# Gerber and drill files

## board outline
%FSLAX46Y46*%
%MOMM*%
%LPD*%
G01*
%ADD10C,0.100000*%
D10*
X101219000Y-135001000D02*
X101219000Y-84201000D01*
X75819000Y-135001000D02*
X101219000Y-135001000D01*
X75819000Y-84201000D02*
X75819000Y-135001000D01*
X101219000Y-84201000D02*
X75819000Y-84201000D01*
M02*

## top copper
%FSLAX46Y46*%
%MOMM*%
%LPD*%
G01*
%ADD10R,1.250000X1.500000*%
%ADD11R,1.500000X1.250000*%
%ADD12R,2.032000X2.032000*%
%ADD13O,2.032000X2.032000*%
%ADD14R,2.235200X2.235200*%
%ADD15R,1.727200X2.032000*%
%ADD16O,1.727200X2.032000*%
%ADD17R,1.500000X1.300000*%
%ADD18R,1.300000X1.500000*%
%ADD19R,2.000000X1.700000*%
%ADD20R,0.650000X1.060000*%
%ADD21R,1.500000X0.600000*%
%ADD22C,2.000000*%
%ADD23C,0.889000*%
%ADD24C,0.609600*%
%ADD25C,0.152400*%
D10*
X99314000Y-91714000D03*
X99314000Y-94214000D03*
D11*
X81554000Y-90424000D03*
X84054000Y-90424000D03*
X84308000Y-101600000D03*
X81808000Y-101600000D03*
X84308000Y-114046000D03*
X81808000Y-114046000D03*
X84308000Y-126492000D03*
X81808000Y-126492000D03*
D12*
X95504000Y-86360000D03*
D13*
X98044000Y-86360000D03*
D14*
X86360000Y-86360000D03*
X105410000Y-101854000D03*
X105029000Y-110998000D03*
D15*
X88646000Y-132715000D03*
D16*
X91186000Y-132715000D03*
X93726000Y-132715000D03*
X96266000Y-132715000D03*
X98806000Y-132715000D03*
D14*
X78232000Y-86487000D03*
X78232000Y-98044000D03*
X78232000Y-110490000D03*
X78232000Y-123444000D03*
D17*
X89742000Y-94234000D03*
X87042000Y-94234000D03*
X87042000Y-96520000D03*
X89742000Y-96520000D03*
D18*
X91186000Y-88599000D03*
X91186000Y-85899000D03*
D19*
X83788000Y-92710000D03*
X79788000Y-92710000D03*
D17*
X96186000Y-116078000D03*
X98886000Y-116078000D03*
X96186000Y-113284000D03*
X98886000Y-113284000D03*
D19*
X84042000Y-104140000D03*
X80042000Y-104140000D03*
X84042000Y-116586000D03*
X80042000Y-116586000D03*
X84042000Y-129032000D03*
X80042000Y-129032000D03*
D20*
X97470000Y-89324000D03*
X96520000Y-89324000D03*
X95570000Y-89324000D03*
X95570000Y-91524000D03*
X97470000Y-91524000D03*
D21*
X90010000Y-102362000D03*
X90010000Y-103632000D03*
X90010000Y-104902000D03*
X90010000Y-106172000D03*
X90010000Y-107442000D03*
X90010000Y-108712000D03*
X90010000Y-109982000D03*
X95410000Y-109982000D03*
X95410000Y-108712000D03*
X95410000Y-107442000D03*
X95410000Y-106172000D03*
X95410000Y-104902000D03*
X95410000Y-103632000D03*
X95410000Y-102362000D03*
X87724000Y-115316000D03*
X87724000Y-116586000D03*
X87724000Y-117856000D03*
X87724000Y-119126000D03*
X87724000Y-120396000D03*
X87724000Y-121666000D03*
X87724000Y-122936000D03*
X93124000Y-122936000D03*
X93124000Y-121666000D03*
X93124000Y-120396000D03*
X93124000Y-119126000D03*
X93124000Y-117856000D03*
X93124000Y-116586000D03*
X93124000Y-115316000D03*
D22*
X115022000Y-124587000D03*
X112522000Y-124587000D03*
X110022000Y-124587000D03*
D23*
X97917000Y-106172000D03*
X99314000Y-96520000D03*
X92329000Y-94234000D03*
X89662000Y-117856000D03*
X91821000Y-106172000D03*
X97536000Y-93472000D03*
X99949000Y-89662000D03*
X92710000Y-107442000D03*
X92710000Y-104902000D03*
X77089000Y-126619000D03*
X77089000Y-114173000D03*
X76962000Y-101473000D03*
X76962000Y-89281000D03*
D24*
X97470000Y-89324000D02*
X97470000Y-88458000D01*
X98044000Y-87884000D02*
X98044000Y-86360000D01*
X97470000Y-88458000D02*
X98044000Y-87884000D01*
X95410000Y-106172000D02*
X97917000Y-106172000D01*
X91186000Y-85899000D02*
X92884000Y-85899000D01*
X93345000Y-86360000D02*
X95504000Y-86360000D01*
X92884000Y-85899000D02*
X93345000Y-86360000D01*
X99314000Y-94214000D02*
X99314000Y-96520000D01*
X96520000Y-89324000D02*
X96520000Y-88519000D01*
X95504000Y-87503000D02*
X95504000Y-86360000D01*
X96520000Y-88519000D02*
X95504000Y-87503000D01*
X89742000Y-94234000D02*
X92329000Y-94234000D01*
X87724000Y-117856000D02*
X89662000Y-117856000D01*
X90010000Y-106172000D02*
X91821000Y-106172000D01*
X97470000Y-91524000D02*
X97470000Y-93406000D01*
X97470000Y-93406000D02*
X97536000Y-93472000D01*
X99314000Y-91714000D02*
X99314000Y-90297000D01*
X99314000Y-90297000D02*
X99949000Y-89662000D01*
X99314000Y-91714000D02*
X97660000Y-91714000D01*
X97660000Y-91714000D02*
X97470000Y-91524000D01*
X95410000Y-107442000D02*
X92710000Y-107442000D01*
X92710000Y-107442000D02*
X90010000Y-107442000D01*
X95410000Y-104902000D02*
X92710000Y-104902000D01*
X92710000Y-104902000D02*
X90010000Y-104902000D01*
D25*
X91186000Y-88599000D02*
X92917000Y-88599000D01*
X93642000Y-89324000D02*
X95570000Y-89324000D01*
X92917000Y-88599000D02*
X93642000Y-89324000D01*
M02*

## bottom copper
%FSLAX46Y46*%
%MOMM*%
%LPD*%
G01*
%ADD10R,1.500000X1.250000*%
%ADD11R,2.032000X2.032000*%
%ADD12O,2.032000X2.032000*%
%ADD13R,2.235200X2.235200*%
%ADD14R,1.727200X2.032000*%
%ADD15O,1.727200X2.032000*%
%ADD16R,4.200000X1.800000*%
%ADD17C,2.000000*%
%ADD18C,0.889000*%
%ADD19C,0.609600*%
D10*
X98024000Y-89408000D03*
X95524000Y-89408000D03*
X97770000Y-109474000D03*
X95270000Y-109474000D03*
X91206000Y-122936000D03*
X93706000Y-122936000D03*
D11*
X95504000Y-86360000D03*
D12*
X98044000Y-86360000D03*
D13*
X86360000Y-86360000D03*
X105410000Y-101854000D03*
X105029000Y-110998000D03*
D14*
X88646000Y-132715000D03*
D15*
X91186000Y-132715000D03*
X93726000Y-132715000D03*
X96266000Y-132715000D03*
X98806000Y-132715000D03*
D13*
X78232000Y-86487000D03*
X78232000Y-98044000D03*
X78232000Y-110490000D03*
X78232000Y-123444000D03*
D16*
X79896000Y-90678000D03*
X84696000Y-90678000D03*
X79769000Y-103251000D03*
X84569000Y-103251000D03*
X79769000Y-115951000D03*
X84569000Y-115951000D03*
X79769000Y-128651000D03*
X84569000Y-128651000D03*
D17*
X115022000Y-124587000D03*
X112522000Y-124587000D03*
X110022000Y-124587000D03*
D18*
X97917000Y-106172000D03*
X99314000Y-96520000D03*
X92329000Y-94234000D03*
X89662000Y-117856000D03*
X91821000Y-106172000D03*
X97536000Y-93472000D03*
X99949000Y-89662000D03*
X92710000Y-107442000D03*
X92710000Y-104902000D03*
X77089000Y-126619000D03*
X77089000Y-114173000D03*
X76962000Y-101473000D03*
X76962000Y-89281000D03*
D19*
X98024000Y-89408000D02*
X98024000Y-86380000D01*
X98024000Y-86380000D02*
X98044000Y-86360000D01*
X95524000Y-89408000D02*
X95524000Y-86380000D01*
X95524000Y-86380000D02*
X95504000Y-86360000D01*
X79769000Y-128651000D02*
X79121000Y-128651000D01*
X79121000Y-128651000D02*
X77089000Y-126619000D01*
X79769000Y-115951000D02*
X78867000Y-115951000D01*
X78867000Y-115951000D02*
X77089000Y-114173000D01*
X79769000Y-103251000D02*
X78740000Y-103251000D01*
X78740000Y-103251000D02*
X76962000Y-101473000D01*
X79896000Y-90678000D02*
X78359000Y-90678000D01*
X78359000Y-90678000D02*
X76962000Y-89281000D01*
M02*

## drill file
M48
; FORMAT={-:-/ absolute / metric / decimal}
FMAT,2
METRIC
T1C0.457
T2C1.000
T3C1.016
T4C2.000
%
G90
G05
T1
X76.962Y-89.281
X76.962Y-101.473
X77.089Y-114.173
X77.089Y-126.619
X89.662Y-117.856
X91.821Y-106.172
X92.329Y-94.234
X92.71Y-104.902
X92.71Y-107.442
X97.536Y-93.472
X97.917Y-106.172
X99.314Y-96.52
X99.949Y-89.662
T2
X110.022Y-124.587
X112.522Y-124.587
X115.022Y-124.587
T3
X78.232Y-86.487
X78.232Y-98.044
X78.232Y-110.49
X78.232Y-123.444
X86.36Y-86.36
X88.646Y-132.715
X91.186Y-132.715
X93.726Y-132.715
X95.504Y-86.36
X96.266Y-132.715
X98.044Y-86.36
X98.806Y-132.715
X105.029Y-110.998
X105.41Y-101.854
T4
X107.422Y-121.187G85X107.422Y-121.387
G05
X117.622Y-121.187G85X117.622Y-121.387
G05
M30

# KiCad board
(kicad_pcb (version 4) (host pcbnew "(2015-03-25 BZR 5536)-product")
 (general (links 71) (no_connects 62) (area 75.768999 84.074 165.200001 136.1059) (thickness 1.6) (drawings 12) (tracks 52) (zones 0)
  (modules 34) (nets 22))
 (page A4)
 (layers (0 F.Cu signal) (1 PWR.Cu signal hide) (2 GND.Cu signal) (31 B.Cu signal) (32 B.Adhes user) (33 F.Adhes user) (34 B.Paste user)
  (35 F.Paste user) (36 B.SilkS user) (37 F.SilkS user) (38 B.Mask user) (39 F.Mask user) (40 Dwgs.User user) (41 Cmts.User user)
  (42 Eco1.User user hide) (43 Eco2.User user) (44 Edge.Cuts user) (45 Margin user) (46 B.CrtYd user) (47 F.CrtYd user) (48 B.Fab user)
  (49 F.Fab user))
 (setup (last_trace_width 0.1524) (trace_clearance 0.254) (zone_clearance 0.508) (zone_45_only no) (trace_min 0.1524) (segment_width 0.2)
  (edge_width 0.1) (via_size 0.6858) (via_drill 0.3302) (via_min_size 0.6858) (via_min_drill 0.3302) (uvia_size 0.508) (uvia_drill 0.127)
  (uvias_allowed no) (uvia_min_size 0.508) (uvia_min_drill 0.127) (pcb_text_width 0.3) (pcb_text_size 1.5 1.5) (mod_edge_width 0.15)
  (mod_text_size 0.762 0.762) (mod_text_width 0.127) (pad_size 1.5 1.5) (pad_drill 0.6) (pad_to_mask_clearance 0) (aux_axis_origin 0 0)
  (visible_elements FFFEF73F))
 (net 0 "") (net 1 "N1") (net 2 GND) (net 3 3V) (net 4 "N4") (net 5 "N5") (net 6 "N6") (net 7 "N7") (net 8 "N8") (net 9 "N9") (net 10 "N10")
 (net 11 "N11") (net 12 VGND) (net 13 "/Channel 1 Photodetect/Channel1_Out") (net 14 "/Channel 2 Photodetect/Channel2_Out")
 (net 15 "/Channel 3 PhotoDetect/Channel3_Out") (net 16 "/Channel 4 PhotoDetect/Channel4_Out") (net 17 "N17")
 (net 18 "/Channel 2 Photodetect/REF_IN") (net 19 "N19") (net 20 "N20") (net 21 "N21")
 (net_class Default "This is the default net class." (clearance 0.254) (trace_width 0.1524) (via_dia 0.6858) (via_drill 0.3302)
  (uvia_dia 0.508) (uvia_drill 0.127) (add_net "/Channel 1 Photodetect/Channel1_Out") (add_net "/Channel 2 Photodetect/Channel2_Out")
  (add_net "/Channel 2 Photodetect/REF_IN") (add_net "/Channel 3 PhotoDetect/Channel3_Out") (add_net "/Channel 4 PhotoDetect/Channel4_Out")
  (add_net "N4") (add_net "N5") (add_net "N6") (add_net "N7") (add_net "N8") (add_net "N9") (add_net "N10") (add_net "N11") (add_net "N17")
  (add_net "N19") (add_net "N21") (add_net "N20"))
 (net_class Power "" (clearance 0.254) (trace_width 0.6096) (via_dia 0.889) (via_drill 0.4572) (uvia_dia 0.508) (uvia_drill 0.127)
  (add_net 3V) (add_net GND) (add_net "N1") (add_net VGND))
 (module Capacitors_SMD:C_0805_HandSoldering (layer B.Cu) (at 96.774 89.408 180)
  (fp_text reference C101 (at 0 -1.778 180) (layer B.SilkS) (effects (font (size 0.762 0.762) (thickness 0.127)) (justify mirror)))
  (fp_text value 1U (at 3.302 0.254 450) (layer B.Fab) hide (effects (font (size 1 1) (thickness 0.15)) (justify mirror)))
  (pad 1 smd rect (at -1.25 0 180) (size 1.5 1.25) (layers B.Cu B.Paste B.Mask) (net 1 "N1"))
  (pad 2 smd rect (at 1.25 0 180) (size 1.5 1.25) (layers B.Cu B.Paste B.Mask) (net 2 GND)))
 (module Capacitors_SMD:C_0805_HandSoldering (layer F.Cu) (at 99.314 92.964 270)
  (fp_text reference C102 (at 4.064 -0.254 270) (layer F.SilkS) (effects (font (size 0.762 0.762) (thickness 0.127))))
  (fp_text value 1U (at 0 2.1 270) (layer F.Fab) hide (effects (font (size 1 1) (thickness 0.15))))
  (pad 1 smd rect (at -1.25 0 270) (size 1.5 1.25) (layers F.Cu F.Paste F.Mask) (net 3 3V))
  (pad 2 smd rect (at 1.25 0 270) (size 1.5 1.25) (layers F.Cu F.Paste F.Mask) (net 2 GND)))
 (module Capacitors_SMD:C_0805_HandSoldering (layer F.Cu) (at 82.804 90.424)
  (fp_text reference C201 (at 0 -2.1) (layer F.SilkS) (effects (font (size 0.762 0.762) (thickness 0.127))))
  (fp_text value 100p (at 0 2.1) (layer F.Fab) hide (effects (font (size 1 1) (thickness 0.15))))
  (pad 1 smd rect (at -1.25 0) (size 1.5 1.25) (layers F.Cu F.Paste F.Mask) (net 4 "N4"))
  (pad 2 smd rect (at 1.25 0) (size 1.5 1.25) (layers F.Cu F.Paste F.Mask) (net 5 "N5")))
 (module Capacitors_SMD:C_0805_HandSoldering (layer B.Cu) (at 96.52 109.474 180)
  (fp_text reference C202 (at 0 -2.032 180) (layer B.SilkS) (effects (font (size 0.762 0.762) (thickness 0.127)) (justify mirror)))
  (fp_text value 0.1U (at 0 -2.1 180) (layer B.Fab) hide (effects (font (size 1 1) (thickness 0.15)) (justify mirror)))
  (pad 1 smd rect (at -1.25 0 180) (size 1.5 1.25) (layers B.Cu B.Paste B.Mask) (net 2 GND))
  (pad 2 smd rect (at 1.25 0 180) (size 1.5 1.25) (layers B.Cu B.Paste B.Mask) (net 3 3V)))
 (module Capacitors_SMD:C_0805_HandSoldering (layer B.Cu) (at 92.456 122.936)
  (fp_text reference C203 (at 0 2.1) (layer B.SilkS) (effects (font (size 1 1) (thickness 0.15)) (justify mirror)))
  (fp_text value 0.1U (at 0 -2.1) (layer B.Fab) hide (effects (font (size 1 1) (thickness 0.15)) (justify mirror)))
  (pad 1 smd rect (at -1.25 0) (size 1.5 1.25) (layers B.Cu B.Paste B.Mask) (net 2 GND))
  (pad 2 smd rect (at 1.25 0) (size 1.5 1.25) (layers B.Cu B.Paste B.Mask) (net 3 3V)))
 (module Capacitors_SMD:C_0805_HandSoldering (layer F.Cu) (at 83.058 101.6 180)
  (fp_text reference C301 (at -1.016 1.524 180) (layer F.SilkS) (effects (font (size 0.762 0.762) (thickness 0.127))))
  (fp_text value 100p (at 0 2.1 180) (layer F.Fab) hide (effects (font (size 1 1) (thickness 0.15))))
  (pad 1 smd rect (at -1.25 0 180) (size 1.5 1.25) (layers F.Cu F.Paste F.Mask) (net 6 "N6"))
  (pad 2 smd rect (at 1.25 0 180) (size 1.5 1.25) (layers F.Cu F.Paste F.Mask) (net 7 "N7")))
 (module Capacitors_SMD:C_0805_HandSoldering (layer F.Cu) (at 83.058 114.046 180)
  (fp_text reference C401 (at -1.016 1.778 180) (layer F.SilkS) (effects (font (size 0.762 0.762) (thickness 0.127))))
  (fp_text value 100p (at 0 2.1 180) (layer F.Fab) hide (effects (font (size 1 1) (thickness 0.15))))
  (pad 1 smd rect (at -1.25 0 180) (size 1.5 1.25) (layers F.Cu F.Paste F.Mask) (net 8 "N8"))
  (pad 2 smd rect (at 1.25 0 180) (size 1.5 1.25) (layers F.Cu F.Paste F.Mask) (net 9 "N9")))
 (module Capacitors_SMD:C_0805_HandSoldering (layer F.Cu) (at 83.058 126.492 180)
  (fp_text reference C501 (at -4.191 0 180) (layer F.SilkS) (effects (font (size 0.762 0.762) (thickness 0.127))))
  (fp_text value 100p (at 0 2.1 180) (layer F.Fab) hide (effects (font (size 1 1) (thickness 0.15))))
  (pad 1 smd rect (at -1.25 0 180) (size 1.5 1.25) (layers F.Cu F.Paste F.Mask) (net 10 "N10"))
  (pad 2 smd rect (at 1.25 0 180) (size 1.5 1.25) (layers F.Cu F.Paste F.Mask) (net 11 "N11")))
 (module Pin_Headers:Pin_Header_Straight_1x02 (layer F.Cu) (at 95.504 86.36 90)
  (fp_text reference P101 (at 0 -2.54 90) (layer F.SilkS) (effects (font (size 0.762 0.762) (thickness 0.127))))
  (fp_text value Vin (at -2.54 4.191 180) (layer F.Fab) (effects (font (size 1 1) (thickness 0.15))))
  (pad 1 thru_hole rect (at 0 0 90) (size 2.032 2.032) (drill 1.016) (layers *.Cu *.Mask F.SilkS) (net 2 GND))
  (pad 2 thru_hole oval (at 0 2.54 90) (size 2.032 2.032) (drill 1.016) (layers *.Cu *.Mask F.SilkS) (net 1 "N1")))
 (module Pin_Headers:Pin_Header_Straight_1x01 (layer F.Cu) (at 86.36 86.36)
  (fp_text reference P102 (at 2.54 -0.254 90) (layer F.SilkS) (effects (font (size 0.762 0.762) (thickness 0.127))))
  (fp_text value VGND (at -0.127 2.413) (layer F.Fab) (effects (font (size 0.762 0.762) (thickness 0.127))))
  (pad 1 thru_hole rect (at 0 0) (size 2.2352 2.2352) (drill 1.016) (layers *.Cu *.Mask F.SilkS) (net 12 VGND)))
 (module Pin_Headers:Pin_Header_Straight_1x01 (layer F.Cu) (at 105.41 101.854)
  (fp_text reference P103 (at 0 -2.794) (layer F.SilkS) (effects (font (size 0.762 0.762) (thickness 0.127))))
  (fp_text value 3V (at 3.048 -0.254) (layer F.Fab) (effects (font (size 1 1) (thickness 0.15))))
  (pad 1 thru_hole rect (at 0 0) (size 2.2352 2.2352) (drill 1.016) (layers *.Cu *.Mask F.SilkS) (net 3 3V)))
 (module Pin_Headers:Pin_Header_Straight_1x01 (layer F.Cu) (at 105.029 110.998)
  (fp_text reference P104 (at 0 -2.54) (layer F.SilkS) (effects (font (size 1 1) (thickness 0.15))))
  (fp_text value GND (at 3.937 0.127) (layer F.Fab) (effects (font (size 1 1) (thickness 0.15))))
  (pad 1 thru_hole rect (at 0 0) (size 2.2352 2.2352) (drill 1.016) (layers *.Cu *.Mask F.SilkS) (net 2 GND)))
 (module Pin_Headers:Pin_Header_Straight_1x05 (layer F.Cu) (at 88.646 132.715 90)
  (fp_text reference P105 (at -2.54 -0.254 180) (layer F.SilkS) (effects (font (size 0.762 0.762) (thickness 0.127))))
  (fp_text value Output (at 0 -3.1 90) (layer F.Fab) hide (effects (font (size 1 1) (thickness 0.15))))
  (pad 1 thru_hole rect (at 0 0 90) (size 2.032 1.7272) (drill 1.016) (layers *.Cu *.Mask F.SilkS)
   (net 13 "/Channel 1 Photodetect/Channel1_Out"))
  (pad 2 thru_hole oval (at 0 2.54 90) (size 2.032 1.7272) (drill 1.016) (layers *.Cu *.Mask F.SilkS)
   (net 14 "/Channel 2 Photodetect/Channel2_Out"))
  (pad 3 thru_hole oval (at 0 5.08 90) (size 2.032 1.7272) (drill 1.016) (layers *.Cu *.Mask F.SilkS)
   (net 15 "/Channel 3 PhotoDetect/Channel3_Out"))
  (pad 4 thru_hole oval (at 0 7.62 90) (size 2.032 1.7272) (drill 1.016) (layers *.Cu *.Mask F.SilkS)
   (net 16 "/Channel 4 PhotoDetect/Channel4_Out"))
  (pad 5 thru_hole oval (at 0 10.16 90) (size 2.032 1.7272) (drill 1.016) (layers *.Cu *.Mask F.SilkS) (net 2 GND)))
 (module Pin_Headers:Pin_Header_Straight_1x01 (layer F.Cu) (at 78.232 86.487)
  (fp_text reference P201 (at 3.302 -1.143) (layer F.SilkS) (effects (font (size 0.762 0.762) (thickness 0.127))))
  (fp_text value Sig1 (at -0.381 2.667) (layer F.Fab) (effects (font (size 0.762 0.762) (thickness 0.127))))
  (pad 1 thru_hole rect (at 0 0) (size 2.2352 2.2352) (drill 1.016) (layers *.Cu *.Mask F.SilkS) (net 4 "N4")))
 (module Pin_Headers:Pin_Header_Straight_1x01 (layer F.Cu) (at 78.232 98.044)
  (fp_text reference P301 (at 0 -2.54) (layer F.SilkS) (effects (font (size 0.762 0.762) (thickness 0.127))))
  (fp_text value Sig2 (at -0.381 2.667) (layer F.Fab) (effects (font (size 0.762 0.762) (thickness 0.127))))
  (pad 1 thru_hole rect (at 0 0) (size 2.2352 2.2352) (drill 1.016) (layers *.Cu *.Mask F.SilkS) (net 6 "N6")))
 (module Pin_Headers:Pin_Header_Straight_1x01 (layer F.Cu) (at 78.232 110.49)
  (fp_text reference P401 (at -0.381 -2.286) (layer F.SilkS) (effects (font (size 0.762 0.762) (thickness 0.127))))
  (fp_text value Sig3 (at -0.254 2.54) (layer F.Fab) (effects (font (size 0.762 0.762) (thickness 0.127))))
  (pad 1 thru_hole rect (at 0 0) (size 2.2352 2.2352) (drill 1.016) (layers *.Cu *.Mask F.SilkS) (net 8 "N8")))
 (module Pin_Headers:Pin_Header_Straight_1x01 (layer F.Cu) (at 78.232 123.444)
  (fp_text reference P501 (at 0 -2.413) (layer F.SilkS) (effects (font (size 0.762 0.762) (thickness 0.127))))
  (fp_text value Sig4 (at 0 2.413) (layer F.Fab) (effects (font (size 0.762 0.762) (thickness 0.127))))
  (pad 1 thru_hole rect (at 0 0) (size 2.2352 2.2352) (drill 1.016) (layers *.Cu *.Mask F.SilkS) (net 10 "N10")))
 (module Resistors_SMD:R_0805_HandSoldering (layer F.Cu) (at 88.392 94.234 180)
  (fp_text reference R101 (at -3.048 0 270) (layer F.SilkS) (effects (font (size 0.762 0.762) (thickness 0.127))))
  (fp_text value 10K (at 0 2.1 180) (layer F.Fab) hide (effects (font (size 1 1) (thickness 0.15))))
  (pad 1 smd rect (at -1.35 0 180) (size 1.5 1.3) (layers F.Cu F.Paste F.Mask) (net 3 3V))
  (pad 2 smd rect (at 1.35 0 180) (size 1.5 1.3) (layers F.Cu F.Paste F.Mask) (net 12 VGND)))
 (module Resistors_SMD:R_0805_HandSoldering (layer F.Cu) (at 88.392 96.52)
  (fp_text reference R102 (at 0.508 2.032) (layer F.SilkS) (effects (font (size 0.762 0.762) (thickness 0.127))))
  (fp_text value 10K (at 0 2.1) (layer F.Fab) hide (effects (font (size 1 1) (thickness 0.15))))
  (pad 1 smd rect (at -1.35 0) (size 1.5 1.3) (layers F.Cu F.Paste F.Mask) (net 12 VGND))
  (pad 2 smd rect (at 1.35 0) (size 1.5 1.3) (layers F.Cu F.Paste F.Mask) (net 2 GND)))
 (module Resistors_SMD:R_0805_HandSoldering (layer F.Cu) (at 91.186 87.249 90)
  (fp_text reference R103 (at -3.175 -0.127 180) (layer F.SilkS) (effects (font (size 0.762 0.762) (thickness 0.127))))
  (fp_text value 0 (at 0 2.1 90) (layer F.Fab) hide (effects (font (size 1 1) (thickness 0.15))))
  (pad 1 smd rect (at -1.35 0 90) (size 1.5 1.3) (layers F.Cu F.Paste F.Mask) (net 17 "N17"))
  (pad 2 smd rect (at 1.35 0 90) (size 1.5 1.3) (layers F.Cu F.Paste F.Mask) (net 2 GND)))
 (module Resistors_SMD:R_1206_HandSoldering (layer F.Cu) (at 81.788 92.71 180)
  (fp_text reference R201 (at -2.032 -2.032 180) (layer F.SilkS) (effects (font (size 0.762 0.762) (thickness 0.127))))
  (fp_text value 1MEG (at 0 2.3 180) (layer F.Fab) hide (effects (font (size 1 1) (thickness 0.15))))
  (pad 1 smd rect (at -2 0 180) (size 2 1.7) (layers F.Cu F.Paste F.Mask) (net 4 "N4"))
  (pad 2 smd rect (at 2 0 180) (size 2 1.7) (layers F.Cu F.Paste F.Mask) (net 5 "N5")))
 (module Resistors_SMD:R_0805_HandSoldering (layer F.Cu) (at 97.536 116.078)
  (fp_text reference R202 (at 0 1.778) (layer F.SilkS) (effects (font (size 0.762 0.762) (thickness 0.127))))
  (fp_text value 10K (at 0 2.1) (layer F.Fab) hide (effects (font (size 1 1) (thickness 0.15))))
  (pad 1 smd rect (at -1.35 0) (size 1.5 1.3) (layers F.Cu F.Paste F.Mask) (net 2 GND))
  (pad 2 smd rect (at 1.35 0) (size 1.5 1.3) (layers F.Cu F.Paste F.Mask) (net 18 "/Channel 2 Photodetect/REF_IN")))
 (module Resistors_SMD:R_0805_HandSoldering (layer F.Cu) (at 97.536 113.284)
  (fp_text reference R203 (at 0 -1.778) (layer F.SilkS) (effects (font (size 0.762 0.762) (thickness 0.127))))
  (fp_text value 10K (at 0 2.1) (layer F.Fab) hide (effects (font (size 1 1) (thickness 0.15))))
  (pad 1 smd rect (at -1.35 0) (size 1.5 1.3) (layers F.Cu F.Paste F.Mask) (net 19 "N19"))
  (pad 2 smd rect (at 1.35 0) (size 1.5 1.3) (layers F.Cu F.Paste F.Mask) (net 3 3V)))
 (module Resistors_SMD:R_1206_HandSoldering (layer F.Cu) (at 82.042 104.14 180)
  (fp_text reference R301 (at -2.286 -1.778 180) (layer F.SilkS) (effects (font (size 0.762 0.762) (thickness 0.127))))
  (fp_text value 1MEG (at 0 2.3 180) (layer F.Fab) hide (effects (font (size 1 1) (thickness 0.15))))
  (pad 1 smd rect (at -2 0 180) (size 2 1.7) (layers F.Cu F.Paste F.Mask) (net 6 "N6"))
  (pad 2 smd rect (at 2 0 180) (size 2 1.7) (layers F.Cu F.Paste F.Mask) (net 7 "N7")))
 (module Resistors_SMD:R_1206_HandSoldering (layer F.Cu) (at 82.042 116.586 180)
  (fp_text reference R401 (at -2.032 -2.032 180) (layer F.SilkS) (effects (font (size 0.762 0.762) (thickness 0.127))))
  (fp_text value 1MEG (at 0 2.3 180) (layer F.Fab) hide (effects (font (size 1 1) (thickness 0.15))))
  (pad 1 smd rect (at -2 0 180) (size 2 1.7) (layers F.Cu F.Paste F.Mask) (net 8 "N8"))
  (pad 2 smd rect (at 2 0 180) (size 2 1.7) (layers F.Cu F.Paste F.Mask) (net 9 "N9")))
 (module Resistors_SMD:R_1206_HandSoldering (layer F.Cu) (at 82.042 129.032 180)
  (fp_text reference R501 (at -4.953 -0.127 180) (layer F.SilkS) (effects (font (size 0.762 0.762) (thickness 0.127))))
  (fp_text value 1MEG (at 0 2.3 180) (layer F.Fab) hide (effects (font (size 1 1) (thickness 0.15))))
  (pad 1 smd rect (at -2 0 180) (size 2 1.7) (layers F.Cu F.Paste F.Mask) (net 10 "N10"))
  (pad 2 smd rect (at 2 0 180) (size 2 1.7) (layers F.Cu F.Paste F.Mask) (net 11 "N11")))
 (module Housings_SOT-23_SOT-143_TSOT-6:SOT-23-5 (layer F.Cu) (at 96.52 90.424 270)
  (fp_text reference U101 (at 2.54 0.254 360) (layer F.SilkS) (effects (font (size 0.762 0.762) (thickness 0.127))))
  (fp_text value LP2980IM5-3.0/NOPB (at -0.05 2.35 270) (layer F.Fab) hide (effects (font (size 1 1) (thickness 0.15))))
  (pad 1 smd rect (at -1.1 -0.95 270) (size 1.06 0.65) (layers F.Cu F.Paste F.Mask) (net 1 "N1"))
  (pad 2 smd rect (at -1.1 0 270) (size 1.06 0.65) (layers F.Cu F.Paste F.Mask) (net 2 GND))
  (pad 3 smd rect (at -1.1 0.95 270) (size 1.06 0.65) (layers F.Cu F.Paste F.Mask) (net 17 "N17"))
  (pad 4 smd rect (at 1.1 0.95 270) (size 1.06 0.65) (layers F.Cu F.Paste F.Mask) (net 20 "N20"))
  (pad 5 smd rect (at 1.1 -0.95 270) (size 1.06 0.65) (layers F.Cu F.Paste F.Mask) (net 3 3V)))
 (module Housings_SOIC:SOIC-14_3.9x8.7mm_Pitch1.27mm (layer F.Cu) (at 92.71 106.172)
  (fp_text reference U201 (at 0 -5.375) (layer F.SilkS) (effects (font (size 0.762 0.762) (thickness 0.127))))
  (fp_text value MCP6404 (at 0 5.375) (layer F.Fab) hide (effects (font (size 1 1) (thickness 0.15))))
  (pad 1 smd rect (at -2.7 -3.81) (size 1.5 0.6) (layers F.Cu F.Paste F.Mask) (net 4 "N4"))
  (pad 2 smd rect (at -2.7 -2.54) (size 1.5 0.6) (layers F.Cu F.Paste F.Mask) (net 5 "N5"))
  (pad 3 smd rect (at -2.7 -1.27) (size 1.5 0.6) (layers F.Cu F.Paste F.Mask) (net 12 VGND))
  (pad 4 smd rect (at -2.7 0) (size 1.5 0.6) (layers F.Cu F.Paste F.Mask) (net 3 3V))
  (pad 5 smd rect (at -2.7 1.27) (size 1.5 0.6) (layers F.Cu F.Paste F.Mask) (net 12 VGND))
  (pad 6 smd rect (at -2.7 2.54) (size 1.5 0.6) (layers F.Cu F.Paste F.Mask) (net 7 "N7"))
  (pad 7 smd rect (at -2.7 3.81) (size 1.5 0.6) (layers F.Cu F.Paste F.Mask) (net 6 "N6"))
  (pad 8 smd rect (at 2.7 3.81) (size 1.5 0.6) (layers F.Cu F.Paste F.Mask) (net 8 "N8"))
  (pad 9 smd rect (at 2.7 2.54) (size 1.5 0.6) (layers F.Cu F.Paste F.Mask) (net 9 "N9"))
  (pad 10 smd rect (at 2.7 1.27) (size 1.5 0.6) (layers F.Cu F.Paste F.Mask) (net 12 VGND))
  (pad 11 smd rect (at 2.7 0) (size 1.5 0.6) (layers F.Cu F.Paste F.Mask) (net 2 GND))
  (pad 12 smd rect (at 2.7 -1.27) (size 1.5 0.6) (layers F.Cu F.Paste F.Mask) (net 12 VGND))
  (pad 13 smd rect (at 2.7 -2.54) (size 1.5 0.6) (layers F.Cu F.Paste F.Mask) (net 11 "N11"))
  (pad 14 smd rect (at 2.7 -3.81) (size 1.5 0.6) (layers F.Cu F.Paste F.Mask) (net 10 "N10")))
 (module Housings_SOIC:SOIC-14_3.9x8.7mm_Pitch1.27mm (layer F.Cu) (at 90.424 119.126)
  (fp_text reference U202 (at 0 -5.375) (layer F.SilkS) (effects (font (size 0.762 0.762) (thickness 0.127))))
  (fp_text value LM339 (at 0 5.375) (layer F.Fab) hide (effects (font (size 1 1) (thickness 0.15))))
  (pad 1 smd rect (at -2.7 -3.81) (size 1.5 0.6) (layers F.Cu F.Paste F.Mask) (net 14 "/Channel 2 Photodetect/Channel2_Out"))
  (pad 2 smd rect (at -2.7 -2.54) (size 1.5 0.6) (layers F.Cu F.Paste F.Mask) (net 13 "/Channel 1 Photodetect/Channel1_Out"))
  (pad 3 smd rect (at -2.7 -1.27) (size 1.5 0.6) (layers F.Cu F.Paste F.Mask) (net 3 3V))
  (pad 4 smd rect (at -2.7 0) (size 1.5 0.6) (layers F.Cu F.Paste F.Mask) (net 18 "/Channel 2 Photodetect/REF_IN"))
  (pad 5 smd rect (at -2.7 1.27) (size 1.5 0.6) (layers F.Cu F.Paste F.Mask) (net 4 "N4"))
  (pad 6 smd rect (at -2.7 2.54) (size 1.5 0.6) (layers F.Cu F.Paste F.Mask) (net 18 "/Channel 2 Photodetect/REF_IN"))
  (pad 7 smd rect (at -2.7 3.81) (size 1.5 0.6) (layers F.Cu F.Paste F.Mask) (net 6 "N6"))
  (pad 8 smd rect (at 2.7 3.81) (size 1.5 0.6) (layers F.Cu F.Paste F.Mask) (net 18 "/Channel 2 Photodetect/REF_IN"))
  (pad 9 smd rect (at 2.7 2.54) (size 1.5 0.6) (layers F.Cu F.Paste F.Mask) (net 10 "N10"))
  (pad 10 smd rect (at 2.7 1.27) (size 1.5 0.6) (layers F.Cu F.Paste F.Mask) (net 18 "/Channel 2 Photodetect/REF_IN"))
  (pad 11 smd rect (at 2.7 0) (size 1.5 0.6) (layers F.Cu F.Paste F.Mask) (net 8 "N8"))
  (pad 12 smd rect (at 2.7 -1.27) (size 1.5 0.6) (layers F.Cu F.Paste F.Mask) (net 2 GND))
  (pad 13 smd rect (at 2.7 -2.54) (size 1.5 0.6) (layers F.Cu F.Paste F.Mask) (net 15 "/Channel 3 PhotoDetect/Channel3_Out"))
  (pad 14 smd rect (at 2.7 -3.81) (size 1.5 0.6) (layers F.Cu F.Paste F.Mask) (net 16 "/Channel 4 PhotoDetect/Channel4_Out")))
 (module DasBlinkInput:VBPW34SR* (layer B.Cu) (at 82.296 90.678)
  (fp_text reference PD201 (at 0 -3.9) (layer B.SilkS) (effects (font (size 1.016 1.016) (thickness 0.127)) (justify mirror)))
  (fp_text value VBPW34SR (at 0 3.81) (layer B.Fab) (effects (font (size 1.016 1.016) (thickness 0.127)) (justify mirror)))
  (pad 1 smd rect (at -2.4 0) (size 4.2 1.8) (layers B.Cu B.Paste B.Mask) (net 12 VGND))
  (pad 2 smd rect (at 2.4 0) (size 4.2 1.8) (layers B.Cu B.Paste B.Mask) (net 5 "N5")))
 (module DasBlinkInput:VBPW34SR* (layer B.Cu) (at 82.169 103.251)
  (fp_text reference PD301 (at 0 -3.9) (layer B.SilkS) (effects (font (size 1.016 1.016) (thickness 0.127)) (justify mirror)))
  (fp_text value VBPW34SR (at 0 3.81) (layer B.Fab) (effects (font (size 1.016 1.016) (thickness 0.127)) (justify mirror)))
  (pad 1 smd rect (at -2.4 0) (size 4.2 1.8) (layers B.Cu B.Paste B.Mask) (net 12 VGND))
  (pad 2 smd rect (at 2.4 0) (size 4.2 1.8) (layers B.Cu B.Paste B.Mask) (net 7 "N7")))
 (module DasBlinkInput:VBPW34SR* (layer B.Cu) (at 82.169 115.951)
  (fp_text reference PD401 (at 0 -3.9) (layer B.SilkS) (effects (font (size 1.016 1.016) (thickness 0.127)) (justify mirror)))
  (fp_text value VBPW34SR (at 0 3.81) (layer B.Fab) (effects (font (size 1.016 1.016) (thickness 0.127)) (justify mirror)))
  (pad 1 smd rect (at -2.4 0) (size 4.2 1.8) (layers B.Cu B.Paste B.Mask) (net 12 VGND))
  (pad 2 smd rect (at 2.4 0) (size 4.2 1.8) (layers B.Cu B.Paste B.Mask) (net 9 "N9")))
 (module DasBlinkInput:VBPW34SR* (layer B.Cu) (at 82.169 128.651)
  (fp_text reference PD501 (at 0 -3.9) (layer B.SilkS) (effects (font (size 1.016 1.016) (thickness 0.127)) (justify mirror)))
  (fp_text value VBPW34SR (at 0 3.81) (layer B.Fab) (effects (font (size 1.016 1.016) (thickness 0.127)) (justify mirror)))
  (pad 1 smd rect (at -2.4 0) (size 4.2 1.8) (layers B.Cu B.Paste B.Mask) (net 12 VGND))
  (pad 2 smd rect (at 2.4 0) (size 4.2 1.8) (layers B.Cu B.Paste B.Mask) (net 11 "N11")))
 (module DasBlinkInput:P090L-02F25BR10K (layer F.Cu) (at 112.522 124.587)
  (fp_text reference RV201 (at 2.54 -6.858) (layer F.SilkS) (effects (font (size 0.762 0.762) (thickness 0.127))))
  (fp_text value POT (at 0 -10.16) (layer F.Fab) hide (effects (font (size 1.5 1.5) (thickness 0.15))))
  (pad 3 thru_hole circle (at 2.5 0) (size 2 2) (drill 1) (layers *.Cu *.Mask F.SilkS) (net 18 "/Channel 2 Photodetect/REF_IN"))
  (pad 2 thru_hole circle (at 0 0) (size 2 2) (drill 1) (layers *.Cu *.Mask F.SilkS) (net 19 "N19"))
  (pad 1 thru_hole circle (at -2.5 0) (size 2 2) (drill 1) (layers *.Cu *.Mask F.SilkS) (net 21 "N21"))
  (pad "" np_thru_hole oval (at 5.1 -3.3) (size 2 2.2) (drill oval 2 2.2) (layers *.Cu *.Mask F.SilkS))
  (pad "" np_thru_hole oval (at -5.1 -3.3) (size 2 2.2) (drill oval 2 2.2) (layers *.Cu *.Mask F.SilkS)))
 (gr_line (start 101.219 135.001) (end 101.219 84.201) (angle 90) (layer Edge.Cuts) (width 0.1))
 (gr_line (start 75.819 135.001) (end 101.219 135.001) (angle 90) (layer Edge.Cuts) (width 0.1))
 (gr_line (start 75.819 84.201) (end 75.819 135.001) (angle 90) (layer Edge.Cuts) (width 0.1))
 (gr_line (start 101.219 84.201) (end 75.819 84.201) (angle 90) (layer Edge.Cuts) (width 0.1))
 (segment (start 97.47 89.324) (end 97.47 88.458) (width 0.6096) (layer F.Cu) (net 1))
 (segment (start 98.044 87.884) (end 98.044 86.36) (width 0.6096) (layer F.Cu) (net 1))
 (segment (start 97.47 88.458) (end 98.044 87.884) (width 0.6096) (layer F.Cu) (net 1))
 (segment (start 98.024 89.408) (end 98.024 86.38) (width 0.6096) (layer B.Cu) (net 1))
 (segment (start 98.024 86.38) (end 98.044 86.36) (width 0.6096) (layer B.Cu) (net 1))
 (segment (start 95.41 106.172) (end 97.917 106.172) (width 0.6096) (layer F.Cu) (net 2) (status 400000))
 (via (at 97.917 106.172) (size 0.889) (layers F.Cu B.Cu) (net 2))
 (segment (start 91.186 85.899) (end 92.884 85.899) (width 0.6096) (layer F.Cu) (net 2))
 (segment (start 93.345 86.36) (end 95.504 86.36) (width 0.6096) (layer F.Cu) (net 2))
 (segment (start 92.884 85.899) (end 93.345 86.36) (width 0.6096) (layer F.Cu) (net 2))
 (segment (start 99.314 94.214) (end 99.314 96.52) (width 0.6096) (layer F.Cu) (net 2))
 (via (at 99.314 96.52) (size 0.889) (layers F.Cu B.Cu) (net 2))
 (segment (start 96.52 89.324) (end 96.52 88.519) (width 0.6096) (layer F.Cu) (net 2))
 (segment (start 95.504 87.503) (end 95.504 86.36) (width 0.6096) (layer F.Cu) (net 2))
 (segment (start 96.52 88.519) (end 95.504 87.503) (width 0.6096) (layer F.Cu) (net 2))
 (segment (start 95.524 89.408) (end 95.524 86.38) (width 0.6096) (layer B.Cu) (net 2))
 (segment (start 95.524 86.38) (end 95.504 86.36) (width 0.6096) (layer B.Cu) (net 2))
 (segment (start 89.742 94.234) (end 92.329 94.234) (width 0.6096) (layer F.Cu) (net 3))
 (via (at 92.329 94.234) (size 0.889) (layers F.Cu B.Cu) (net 3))
 (segment (start 87.724 117.856) (end 89.662 117.856) (width 0.6096) (layer F.Cu) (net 3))
 (via (at 89.662 117.856) (size 0.889) (layers F.Cu B.Cu) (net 3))
 (segment (start 90.01 106.172) (end 91.821 106.172) (width 0.6096) (layer F.Cu) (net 3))
 (via (at 91.821 106.172) (size 0.889) (layers F.Cu B.Cu) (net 3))
 (segment (start 97.47 91.524) (end 97.47 93.406) (width 0.6096) (layer F.Cu) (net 3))
 (via (at 97.536 93.472) (size 0.889) (layers F.Cu B.Cu) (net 3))
 (segment (start 97.47 93.406) (end 97.536 93.472) (width 0.6096) (layer F.Cu) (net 3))
 (segment (start 99.314 91.714) (end 99.314 90.297) (width 0.6096) (layer F.Cu) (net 3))
 (via (at 99.949 89.662) (size 0.889) (layers F.Cu B.Cu) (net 3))
 (segment (start 99.314 90.297) (end 99.949 89.662) (width 0.6096) (layer F.Cu) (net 3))
 (segment (start 99.314 91.714) (end 97.66 91.714) (width 0.6096) (layer F.Cu) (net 3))
 (segment (start 97.66 91.714) (end 97.47 91.524) (width 0.6096) (layer F.Cu) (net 3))
 (segment (start 95.41 107.442) (end 92.71 107.442) (width 0.6096) (layer F.Cu) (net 12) (status 400000))
 (via (at 92.71 107.442) (size 0.889) (layers F.Cu B.Cu) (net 12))
 (segment (start 92.71 107.442) (end 90.01 107.442) (width 0.6096) (layer F.Cu) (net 12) (status 800000))
 (segment (start 95.41 104.902) (end 92.71 104.902) (width 0.6096) (layer F.Cu) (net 12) (status 400000))
 (via (at 92.71 104.902) (size 0.889) (layers F.Cu B.Cu) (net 12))
 (segment (start 92.71 104.902) (end 90.01 104.902) (width 0.6096) (layer F.Cu) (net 12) (status 800000))
 (segment (start 79.769 128.651) (end 79.121 128.651) (width 0.6096) (layer B.Cu) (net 12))
 (segment (start 79.121 128.651) (end 77.089 126.619) (width 0.6096) (layer B.Cu) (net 12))
 (via (at 77.089 126.619) (size 0.889) (layers F.Cu B.Cu) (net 12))
 (segment (start 79.769 115.951) (end 78.867 115.951) (width 0.6096) (layer B.Cu) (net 12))
 (segment (start 78.867 115.951) (end 77.089 114.173) (width 0.6096) (layer B.Cu) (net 12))
 (via (at 77.089 114.173) (size 0.889) (layers F.Cu B.Cu) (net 12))
 (segment (start 79.769 103.251) (end 78.74 103.251) (width 0.6096) (layer B.Cu) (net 12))
 (segment (start 78.74 103.251) (end 76.962 101.473) (width 0.6096) (layer B.Cu) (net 12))
 (via (at 76.962 101.473) (size 0.889) (layers F.Cu B.Cu) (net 12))
 (segment (start 79.896 90.678) (end 78.359 90.678) (width 0.6096) (layer B.Cu) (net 12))
 (segment (start 78.359 90.678) (end 76.962 89.281) (width 0.6096) (layer B.Cu) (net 12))
 (via (at 76.962 89.281) (size 0.889) (layers F.Cu B.Cu) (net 12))
 (segment (start 91.186 88.599) (end 92.917 88.599) (width 0.1524) (layer F.Cu) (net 17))
 (segment (start 93.642 89.324) (end 95.57 89.324) (width 0.1524) (layer F.Cu) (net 17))
 (segment (start 92.917 88.599) (end 93.642 89.324) (width 0.1524) (layer F.Cu) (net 17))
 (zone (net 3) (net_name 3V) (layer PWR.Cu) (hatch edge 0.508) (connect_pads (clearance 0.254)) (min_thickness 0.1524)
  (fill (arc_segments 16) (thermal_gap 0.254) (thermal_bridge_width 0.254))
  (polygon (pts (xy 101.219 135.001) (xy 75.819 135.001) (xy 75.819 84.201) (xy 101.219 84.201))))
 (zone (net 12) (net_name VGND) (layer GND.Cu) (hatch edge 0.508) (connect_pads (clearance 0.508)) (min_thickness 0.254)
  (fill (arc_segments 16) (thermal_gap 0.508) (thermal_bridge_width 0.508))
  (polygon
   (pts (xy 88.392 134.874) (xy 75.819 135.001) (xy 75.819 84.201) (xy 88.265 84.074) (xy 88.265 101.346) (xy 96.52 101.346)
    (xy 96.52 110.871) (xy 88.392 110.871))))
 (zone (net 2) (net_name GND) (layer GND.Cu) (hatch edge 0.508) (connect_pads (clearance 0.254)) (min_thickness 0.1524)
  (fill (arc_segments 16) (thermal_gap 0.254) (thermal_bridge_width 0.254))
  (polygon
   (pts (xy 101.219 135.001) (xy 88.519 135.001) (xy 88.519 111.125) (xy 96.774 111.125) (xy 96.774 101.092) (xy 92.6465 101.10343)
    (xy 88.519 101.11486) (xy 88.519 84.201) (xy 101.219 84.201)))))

